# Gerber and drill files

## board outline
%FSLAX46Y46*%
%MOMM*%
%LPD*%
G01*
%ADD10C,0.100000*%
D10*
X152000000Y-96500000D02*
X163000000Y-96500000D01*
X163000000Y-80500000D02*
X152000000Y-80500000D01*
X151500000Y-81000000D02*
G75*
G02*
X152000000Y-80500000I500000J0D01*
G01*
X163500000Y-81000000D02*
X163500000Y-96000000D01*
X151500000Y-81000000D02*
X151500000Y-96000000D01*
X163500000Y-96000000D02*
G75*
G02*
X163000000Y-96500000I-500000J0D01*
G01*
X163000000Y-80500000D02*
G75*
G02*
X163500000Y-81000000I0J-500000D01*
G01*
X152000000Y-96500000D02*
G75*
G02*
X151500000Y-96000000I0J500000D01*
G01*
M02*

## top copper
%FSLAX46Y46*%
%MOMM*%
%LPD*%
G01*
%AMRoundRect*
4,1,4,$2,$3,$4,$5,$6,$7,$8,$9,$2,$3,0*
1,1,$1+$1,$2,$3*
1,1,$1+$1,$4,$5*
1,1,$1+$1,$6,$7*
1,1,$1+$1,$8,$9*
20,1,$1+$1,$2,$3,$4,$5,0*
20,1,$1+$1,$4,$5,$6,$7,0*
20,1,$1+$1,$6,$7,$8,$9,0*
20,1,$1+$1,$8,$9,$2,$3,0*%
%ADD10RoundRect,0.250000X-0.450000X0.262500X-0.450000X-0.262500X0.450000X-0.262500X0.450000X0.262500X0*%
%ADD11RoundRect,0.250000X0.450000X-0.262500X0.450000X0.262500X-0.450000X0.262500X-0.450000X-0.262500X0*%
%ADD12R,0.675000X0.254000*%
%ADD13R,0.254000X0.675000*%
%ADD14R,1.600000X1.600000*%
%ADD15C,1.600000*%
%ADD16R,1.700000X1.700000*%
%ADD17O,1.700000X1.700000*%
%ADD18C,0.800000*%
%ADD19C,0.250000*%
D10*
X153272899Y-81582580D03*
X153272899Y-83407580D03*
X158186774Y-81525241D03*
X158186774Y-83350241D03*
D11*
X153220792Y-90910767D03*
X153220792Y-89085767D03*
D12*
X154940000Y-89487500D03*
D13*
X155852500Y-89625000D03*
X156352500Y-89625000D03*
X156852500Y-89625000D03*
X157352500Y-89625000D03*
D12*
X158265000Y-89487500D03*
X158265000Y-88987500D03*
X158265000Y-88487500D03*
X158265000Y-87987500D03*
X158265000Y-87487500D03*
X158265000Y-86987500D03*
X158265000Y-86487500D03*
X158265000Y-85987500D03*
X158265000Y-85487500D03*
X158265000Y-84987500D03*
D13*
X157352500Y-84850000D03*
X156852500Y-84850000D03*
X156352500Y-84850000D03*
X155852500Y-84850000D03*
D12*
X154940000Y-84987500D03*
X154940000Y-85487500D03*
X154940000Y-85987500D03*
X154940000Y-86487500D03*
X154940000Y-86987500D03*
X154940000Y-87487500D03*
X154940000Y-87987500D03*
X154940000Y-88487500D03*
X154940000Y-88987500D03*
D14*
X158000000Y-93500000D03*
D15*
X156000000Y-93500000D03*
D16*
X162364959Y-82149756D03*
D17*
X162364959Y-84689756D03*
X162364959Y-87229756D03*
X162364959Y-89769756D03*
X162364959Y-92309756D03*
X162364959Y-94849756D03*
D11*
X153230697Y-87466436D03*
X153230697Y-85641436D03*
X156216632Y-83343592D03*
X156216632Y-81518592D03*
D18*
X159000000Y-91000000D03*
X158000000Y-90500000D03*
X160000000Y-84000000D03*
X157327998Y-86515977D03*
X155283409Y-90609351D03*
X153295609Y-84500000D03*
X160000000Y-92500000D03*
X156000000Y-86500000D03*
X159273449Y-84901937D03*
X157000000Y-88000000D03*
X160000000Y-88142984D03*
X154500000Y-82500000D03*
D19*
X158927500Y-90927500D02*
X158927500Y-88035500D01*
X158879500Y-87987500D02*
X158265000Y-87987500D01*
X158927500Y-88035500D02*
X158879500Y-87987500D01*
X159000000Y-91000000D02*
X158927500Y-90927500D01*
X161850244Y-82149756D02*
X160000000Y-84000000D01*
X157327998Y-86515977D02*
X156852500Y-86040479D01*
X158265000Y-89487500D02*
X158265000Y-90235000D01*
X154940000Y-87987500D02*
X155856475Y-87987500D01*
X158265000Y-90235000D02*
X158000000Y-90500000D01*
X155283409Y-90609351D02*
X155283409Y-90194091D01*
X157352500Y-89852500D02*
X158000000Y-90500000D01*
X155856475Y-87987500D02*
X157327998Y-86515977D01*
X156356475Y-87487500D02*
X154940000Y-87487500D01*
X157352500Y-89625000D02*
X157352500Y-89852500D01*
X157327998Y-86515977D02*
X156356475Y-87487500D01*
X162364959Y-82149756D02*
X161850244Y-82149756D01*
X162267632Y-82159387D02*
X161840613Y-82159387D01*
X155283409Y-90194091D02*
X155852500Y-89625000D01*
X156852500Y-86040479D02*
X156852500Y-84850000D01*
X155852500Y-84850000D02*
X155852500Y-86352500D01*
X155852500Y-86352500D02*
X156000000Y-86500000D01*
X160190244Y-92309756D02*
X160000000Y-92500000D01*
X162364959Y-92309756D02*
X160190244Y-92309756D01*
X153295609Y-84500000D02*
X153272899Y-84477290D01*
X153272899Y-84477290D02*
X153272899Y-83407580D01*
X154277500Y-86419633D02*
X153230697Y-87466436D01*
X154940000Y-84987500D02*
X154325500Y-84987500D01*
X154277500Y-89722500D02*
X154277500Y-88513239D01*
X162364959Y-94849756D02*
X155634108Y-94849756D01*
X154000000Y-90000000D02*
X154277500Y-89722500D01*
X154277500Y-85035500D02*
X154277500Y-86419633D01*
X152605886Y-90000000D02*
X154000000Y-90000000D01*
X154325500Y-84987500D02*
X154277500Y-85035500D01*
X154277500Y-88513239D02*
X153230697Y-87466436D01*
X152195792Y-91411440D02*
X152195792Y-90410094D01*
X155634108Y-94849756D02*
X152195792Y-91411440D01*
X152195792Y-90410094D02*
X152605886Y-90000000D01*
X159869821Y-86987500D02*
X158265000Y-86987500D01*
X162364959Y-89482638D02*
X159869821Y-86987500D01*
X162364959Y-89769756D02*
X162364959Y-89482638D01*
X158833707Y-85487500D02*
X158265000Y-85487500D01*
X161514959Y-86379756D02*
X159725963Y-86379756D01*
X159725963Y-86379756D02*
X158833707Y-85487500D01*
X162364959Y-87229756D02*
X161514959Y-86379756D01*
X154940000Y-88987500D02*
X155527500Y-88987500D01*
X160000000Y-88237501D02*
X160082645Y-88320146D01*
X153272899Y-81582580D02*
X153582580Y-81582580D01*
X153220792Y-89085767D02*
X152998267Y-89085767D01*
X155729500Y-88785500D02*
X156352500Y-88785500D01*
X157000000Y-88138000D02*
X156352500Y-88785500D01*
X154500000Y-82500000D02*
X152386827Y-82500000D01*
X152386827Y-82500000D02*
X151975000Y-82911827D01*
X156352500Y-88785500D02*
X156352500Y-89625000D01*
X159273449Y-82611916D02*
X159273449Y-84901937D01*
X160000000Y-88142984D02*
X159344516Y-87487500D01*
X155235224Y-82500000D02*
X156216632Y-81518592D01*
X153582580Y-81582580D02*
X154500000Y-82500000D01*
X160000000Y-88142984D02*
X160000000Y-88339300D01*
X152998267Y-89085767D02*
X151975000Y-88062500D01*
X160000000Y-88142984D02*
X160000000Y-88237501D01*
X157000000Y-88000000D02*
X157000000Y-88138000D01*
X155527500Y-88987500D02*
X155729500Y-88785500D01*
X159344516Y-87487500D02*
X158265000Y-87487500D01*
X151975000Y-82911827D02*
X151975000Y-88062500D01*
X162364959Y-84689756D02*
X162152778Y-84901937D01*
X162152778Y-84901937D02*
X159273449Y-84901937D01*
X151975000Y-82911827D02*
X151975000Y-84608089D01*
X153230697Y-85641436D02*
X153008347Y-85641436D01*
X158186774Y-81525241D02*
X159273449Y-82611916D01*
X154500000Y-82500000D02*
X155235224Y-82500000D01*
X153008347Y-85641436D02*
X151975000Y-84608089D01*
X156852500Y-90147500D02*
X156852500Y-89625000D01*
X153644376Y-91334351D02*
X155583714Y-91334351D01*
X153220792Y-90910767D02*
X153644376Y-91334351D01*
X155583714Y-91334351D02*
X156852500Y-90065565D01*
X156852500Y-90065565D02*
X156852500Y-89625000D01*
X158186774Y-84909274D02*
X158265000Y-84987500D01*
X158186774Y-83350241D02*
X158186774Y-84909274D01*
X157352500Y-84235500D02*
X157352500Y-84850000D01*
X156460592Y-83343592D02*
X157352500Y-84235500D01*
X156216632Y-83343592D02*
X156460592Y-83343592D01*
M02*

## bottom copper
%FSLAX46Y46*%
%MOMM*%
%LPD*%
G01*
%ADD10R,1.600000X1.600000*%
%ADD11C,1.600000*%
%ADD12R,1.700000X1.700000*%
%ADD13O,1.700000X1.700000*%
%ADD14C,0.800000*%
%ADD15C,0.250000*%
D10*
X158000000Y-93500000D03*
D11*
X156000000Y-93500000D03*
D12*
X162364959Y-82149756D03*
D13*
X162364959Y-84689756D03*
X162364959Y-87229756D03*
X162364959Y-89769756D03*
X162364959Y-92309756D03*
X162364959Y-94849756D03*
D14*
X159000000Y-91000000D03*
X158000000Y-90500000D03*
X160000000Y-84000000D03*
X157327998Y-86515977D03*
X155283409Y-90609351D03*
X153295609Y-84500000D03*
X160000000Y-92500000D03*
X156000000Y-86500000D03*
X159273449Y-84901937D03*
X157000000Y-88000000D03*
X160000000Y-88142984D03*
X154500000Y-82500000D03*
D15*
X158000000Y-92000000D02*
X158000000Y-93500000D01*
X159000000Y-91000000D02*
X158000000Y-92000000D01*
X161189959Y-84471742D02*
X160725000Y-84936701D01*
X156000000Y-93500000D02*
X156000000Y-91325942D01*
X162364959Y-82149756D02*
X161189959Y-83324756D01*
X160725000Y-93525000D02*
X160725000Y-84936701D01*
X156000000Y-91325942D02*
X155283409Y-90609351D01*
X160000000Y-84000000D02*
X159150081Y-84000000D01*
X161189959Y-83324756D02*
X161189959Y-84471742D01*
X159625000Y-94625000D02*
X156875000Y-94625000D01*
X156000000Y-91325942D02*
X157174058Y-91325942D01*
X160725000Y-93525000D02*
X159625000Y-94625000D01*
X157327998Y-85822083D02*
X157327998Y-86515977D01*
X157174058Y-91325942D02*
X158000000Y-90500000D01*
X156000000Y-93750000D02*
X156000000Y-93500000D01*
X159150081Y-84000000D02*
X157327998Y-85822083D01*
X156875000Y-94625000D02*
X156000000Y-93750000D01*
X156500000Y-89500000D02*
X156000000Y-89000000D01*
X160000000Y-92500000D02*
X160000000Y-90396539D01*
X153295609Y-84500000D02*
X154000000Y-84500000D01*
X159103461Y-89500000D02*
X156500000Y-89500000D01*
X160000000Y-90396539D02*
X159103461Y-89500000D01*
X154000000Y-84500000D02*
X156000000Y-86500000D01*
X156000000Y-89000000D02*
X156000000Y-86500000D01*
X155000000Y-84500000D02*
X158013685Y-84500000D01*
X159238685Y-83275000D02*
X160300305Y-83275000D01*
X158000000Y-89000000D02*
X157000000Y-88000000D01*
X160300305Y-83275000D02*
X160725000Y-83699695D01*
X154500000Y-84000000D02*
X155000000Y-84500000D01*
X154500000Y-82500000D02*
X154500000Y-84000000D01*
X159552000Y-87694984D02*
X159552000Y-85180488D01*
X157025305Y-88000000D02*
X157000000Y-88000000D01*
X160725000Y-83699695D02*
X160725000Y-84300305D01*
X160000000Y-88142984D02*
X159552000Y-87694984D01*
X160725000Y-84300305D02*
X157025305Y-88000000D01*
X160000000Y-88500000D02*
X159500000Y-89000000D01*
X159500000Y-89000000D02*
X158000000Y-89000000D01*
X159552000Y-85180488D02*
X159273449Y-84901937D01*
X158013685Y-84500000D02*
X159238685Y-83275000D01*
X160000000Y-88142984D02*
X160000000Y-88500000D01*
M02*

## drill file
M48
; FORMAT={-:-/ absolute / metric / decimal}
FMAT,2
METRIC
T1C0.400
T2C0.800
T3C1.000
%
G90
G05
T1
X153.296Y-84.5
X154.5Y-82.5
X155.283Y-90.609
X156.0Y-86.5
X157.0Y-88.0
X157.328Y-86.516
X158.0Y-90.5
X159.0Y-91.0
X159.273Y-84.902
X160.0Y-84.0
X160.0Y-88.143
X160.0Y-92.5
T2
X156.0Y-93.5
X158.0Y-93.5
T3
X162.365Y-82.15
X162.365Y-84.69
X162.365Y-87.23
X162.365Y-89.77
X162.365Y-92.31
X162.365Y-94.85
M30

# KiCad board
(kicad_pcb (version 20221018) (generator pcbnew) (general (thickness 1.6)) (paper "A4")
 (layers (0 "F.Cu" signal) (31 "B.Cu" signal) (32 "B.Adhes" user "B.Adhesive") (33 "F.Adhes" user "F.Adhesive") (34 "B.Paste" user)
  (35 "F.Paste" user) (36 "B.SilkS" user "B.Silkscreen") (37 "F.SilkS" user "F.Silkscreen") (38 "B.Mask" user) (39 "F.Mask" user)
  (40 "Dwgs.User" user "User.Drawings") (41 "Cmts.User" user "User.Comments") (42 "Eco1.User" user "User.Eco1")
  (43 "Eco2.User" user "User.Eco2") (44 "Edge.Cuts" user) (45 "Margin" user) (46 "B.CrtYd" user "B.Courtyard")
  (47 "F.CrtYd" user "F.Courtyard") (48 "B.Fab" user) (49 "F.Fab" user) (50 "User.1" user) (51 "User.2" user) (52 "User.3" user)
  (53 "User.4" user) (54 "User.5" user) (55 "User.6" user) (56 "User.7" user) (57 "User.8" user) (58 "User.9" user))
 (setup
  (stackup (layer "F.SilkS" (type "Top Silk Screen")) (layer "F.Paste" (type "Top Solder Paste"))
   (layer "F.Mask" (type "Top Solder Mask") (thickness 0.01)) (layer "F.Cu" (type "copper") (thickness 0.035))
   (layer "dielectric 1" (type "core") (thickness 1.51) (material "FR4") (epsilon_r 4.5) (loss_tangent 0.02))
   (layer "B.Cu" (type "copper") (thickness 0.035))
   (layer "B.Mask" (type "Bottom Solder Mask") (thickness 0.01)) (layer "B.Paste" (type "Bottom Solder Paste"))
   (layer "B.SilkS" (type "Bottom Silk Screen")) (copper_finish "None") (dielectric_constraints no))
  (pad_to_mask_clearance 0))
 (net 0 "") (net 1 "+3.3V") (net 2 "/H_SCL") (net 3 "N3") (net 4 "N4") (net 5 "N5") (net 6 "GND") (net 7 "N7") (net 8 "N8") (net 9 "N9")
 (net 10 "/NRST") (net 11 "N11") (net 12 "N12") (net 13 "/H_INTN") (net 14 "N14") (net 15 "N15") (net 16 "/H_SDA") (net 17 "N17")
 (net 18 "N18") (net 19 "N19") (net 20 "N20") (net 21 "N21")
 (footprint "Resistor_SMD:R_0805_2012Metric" (layer "F.Cu") (at 153.272899 82.49508 -90)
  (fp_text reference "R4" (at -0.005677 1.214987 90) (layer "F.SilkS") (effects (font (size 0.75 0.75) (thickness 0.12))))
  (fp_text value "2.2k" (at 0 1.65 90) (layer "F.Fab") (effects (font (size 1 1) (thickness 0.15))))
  (pad "1" smd roundrect (at -0.9125 0 270) (size 1.025 1.4) (layers "F.Cu" "F.Paste" "F.Mask") (roundrect_rratio 0.243902) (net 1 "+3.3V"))
  (pad "2" smd roundrect (at 0.9125 0 270) (size 1.025 1.4) (layers "F.Cu" "F.Paste" "F.Mask") (roundrect_rratio 0.243902) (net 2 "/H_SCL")))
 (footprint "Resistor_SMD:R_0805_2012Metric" (layer "F.Cu") (at 158.186774 82.437741 -90)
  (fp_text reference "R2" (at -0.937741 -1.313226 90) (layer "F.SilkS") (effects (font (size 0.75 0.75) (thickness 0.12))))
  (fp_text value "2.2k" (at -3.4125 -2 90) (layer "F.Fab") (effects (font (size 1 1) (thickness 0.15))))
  (pad "1" smd roundrect (at -0.9125 0 270) (size 1.025 1.4) (layers "F.Cu" "F.Paste" "F.Mask") (roundrect_rratio 0.243902) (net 1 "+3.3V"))
  (pad "2" smd roundrect (at 0.9125 0 270) (size 1.025 1.4) (layers "F.Cu" "F.Paste" "F.Mask") (roundrect_rratio 0.243902) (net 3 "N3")))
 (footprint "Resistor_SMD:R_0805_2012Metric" (layer "F.Cu") (at 153.220792 89.998267 90)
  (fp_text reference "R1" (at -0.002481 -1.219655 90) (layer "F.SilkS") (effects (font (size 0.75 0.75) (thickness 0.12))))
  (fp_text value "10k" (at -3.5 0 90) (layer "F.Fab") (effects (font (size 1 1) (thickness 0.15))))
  (pad "1" smd roundrect (at -0.9125 0 90) (size 1.025 1.4) (layers "F.Cu" "F.Paste" "F.Mask") (roundrect_rratio 0.243902) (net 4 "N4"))
  (pad "2" smd roundrect (at 0.9125 0 90) (size 1.025 1.4) (layers "F.Cu" "F.Paste" "F.Mask") (roundrect_rratio 0.243902) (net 1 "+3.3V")))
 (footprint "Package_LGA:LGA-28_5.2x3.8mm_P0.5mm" (layer "F.Cu") (at 156.6025 87.2375 90)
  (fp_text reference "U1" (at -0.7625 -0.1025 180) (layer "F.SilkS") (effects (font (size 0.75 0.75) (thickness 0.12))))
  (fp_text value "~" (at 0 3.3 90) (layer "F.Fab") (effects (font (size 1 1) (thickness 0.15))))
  (pad "1" smd rect (at -2.25 -1.6625 90) (size 0.254 0.675) (layers "F.Cu" "F.Paste" "F.Mask") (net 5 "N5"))
  (pad "2" smd rect (at -2.3875 -0.75 180) (size 0.254 0.675) (layers "F.Cu" "F.Paste" "F.Mask") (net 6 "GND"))
  (pad "3" smd rect (at -2.3875 -0.25 180) (size 0.254 0.675) (layers "F.Cu" "F.Paste" "F.Mask") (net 1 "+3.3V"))
  (pad "4" smd rect (at -2.3875 0.25 180) (size 0.254 0.675) (layers "F.Cu" "F.Paste" "F.Mask") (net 4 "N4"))
  (pad "5" smd rect (at -2.3875 0.75 180) (size 0.254 0.675) (layers "F.Cu" "F.Paste" "F.Mask") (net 6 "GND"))
  (pad "6" smd rect (at -2.25 1.6625 90) (size 0.254 0.675) (layers "F.Cu" "F.Paste" "F.Mask") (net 6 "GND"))
  (pad "7" smd rect (at -1.75 1.6625 90) (size 0.254 0.675) (layers "F.Cu" "F.Paste" "F.Mask") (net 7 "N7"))
  (pad "8" smd rect (at -1.25 1.6625 90) (size 0.254 0.675) (layers "F.Cu" "F.Paste" "F.Mask") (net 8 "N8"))
  (pad "9" smd rect (at -0.75 1.6625 90) (size 0.254 0.675) (layers "F.Cu" "F.Paste" "F.Mask") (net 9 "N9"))
  (pad "10" smd rect (at -0.25 1.6625 90) (size 0.254 0.675) (layers "F.Cu" "F.Paste" "F.Mask") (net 1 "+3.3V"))
  (pad "11" smd rect (at 0.25 1.6625 90) (size 0.254 0.675) (layers "F.Cu" "F.Paste" "F.Mask") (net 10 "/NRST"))
  (pad "12" smd rect (at 0.75 1.6625 90) (size 0.254 0.675) (layers "F.Cu" "F.Paste" "F.Mask") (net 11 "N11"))
  (pad "13" smd rect (at 1.25 1.6625 90) (size 0.254 0.675) (layers "F.Cu" "F.Paste" "F.Mask") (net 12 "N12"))
  (pad "14" smd rect (at 1.75 1.6625 90) (size 0.254 0.675) (layers "F.Cu" "F.Paste" "F.Mask") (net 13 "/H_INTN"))
  (pad "15" smd rect (at 2.25 1.6625 90) (size 0.254 0.675) (layers "F.Cu" "F.Paste" "F.Mask") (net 3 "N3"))
  (pad "16" smd rect (at 2.3875 0.75 180) (size 0.254 0.675) (layers "F.Cu" "F.Paste" "F.Mask") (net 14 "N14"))
  (pad "17" smd rect (at 2.3875 0.25 180) (size 0.254 0.675) (layers "F.Cu" "F.Paste" "F.Mask") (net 6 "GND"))
  (pad "18" smd rect (at 2.3875 -0.25 180) (size 0.254 0.675) (layers "F.Cu" "F.Paste" "F.Mask") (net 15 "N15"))
  (pad "19" smd rect (at 2.3875 -0.75 180) (size 0.254 0.675) (layers "F.Cu" "F.Paste" "F.Mask") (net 2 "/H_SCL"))
  (pad "20" smd rect (at 2.25 -1.6625 90) (size 0.254 0.675) (layers "F.Cu" "F.Paste" "F.Mask") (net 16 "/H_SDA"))
  (pad "21" smd rect (at 1.75 -1.6625 90) (size 0.254 0.675) (layers "F.Cu" "F.Paste" "F.Mask") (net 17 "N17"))
  (pad "22" smd rect (at 1.25 -1.6625 90) (size 0.254 0.675) (layers "F.Cu" "F.Paste" "F.Mask") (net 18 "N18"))
  (pad "23" smd rect (at 0.75 -1.6625 90) (size 0.254 0.675) (layers "F.Cu" "F.Paste" "F.Mask") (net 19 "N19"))
  (pad "24" smd rect (at 0.25 -1.6625 90) (size 0.254 0.675) (layers "F.Cu" "F.Paste" "F.Mask") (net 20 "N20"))
  (pad "25" smd rect (at -0.25 -1.6625 90) (size 0.254 0.675) (layers "F.Cu" "F.Paste" "F.Mask") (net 6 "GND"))
  (pad "26" smd rect (at -0.75 -1.6625 90) (size 0.254 0.675) (layers "F.Cu" "F.Paste" "F.Mask") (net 6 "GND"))
  (pad "27" smd rect (at -1.25 -1.6625 90) (size 0.254 0.675) (layers "F.Cu" "F.Paste" "F.Mask") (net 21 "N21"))
  (pad "28" smd rect (at -1.75 -1.6625 90) (size 0.254 0.675) (layers "F.Cu" "F.Paste" "F.Mask") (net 1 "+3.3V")))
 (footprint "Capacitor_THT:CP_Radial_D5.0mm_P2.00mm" (layer "F.Cu") (at 158 93.5 180)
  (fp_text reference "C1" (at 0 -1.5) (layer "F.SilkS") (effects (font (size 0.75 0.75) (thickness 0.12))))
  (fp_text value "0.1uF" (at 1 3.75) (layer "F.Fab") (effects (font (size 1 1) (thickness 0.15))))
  (pad "1" thru_hole rect (at 0 0 180) (size 1.6 1.6) (drill 0.8) (layers "*.Cu" "*.Mask") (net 9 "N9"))
  (pad "2" thru_hole circle (at 2 0 180) (size 1.6 1.6) (drill 0.8) (layers "*.Cu" "*.Mask") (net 6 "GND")))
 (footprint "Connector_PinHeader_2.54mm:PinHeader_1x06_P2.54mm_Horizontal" (layer "F.Cu") (at 162.364959 82.149756)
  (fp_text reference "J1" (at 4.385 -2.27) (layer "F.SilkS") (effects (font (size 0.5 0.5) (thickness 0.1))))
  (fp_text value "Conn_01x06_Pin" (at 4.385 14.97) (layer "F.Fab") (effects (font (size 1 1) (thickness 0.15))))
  (pad "1" thru_hole rect (at 0 0) (size 1.7 1.7) (drill 1) (layers "*.Cu" "*.Mask") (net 6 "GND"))
  (pad "2" thru_hole oval (at 0 2.54) (size 1.7 1.7) (drill 1) (layers "*.Cu" "*.Mask") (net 1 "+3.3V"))
  (pad "3" thru_hole oval (at 0 5.08) (size 1.7 1.7) (drill 1) (layers "*.Cu" "*.Mask") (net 13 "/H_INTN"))
  (pad "4" thru_hole oval (at 0 7.62) (size 1.7 1.7) (drill 1) (layers "*.Cu" "*.Mask") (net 10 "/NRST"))
  (pad "5" thru_hole oval (at 0 10.16) (size 1.7 1.7) (drill 1) (layers "*.Cu" "*.Mask") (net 2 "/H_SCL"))
  (pad "6" thru_hole oval (at 0 12.7) (size 1.7 1.7) (drill 1) (layers "*.Cu" "*.Mask") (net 16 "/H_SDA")))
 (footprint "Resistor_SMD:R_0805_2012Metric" (layer "F.Cu") (at 153.230697 86.553936 90)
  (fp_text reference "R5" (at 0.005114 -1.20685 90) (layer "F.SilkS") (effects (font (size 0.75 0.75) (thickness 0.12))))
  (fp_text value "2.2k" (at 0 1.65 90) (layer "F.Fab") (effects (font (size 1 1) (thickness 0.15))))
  (pad "1" smd roundrect (at -0.9125 0 90) (size 1.025 1.4) (layers "F.Cu" "F.Paste" "F.Mask") (roundrect_rratio 0.243902) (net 16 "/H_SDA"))
  (pad "2" smd roundrect (at 0.9125 0 90) (size 1.025 1.4) (layers "F.Cu" "F.Paste" "F.Mask") (roundrect_rratio 0.243902) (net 1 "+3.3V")))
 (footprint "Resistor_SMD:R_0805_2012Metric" (layer "F.Cu") (at 156.216632 82.431092 90)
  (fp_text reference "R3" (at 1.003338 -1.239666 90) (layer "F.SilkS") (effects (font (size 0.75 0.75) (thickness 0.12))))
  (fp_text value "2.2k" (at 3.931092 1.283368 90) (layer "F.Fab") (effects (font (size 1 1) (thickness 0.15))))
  (pad "1" smd roundrect (at -0.9125 0 90) (size 1.025 1.4) (layers "F.Cu" "F.Paste" "F.Mask") (roundrect_rratio 0.243902) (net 14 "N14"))
  (pad "2" smd roundrect (at 0.9125 0 90) (size 1.025 1.4) (layers "F.Cu" "F.Paste" "F.Mask") (roundrect_rratio 0.243902) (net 1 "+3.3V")))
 (gr_line (start 152 96.5) (end 163 96.5) (stroke (width 0.1) (type default)) (layer "Edge.Cuts"))
 (gr_line (start 163 80.5) (end 152 80.5) (stroke (width 0.1) (type default)) (layer "Edge.Cuts"))
 (gr_arc (start 151.5 81) (mid 151.646447 80.646447) (end 152 80.5) (stroke (width 0.1) (type default)) (layer "Edge.Cuts"))
 (gr_line (start 163.5 81) (end 163.5 96) (stroke (width 0.1) (type default)) (layer "Edge.Cuts"))
 (gr_line (start 151.5 81) (end 151.5 96) (stroke (width 0.1) (type default)) (layer "Edge.Cuts"))
 (gr_arc (start 163.5 96) (mid 163.353553 96.353553) (end 163 96.5) (stroke (width 0.1) (type default)) (layer "Edge.Cuts"))
 (gr_arc (start 163 80.5) (mid 163.353553 80.646447) (end 163.5 81) (stroke (width 0.1) (type default)) (layer "Edge.Cuts"))
 (gr_arc (start 152 96.5) (mid 151.646447 96.353553) (end 151.5 96) (stroke (width 0.1) (type default)) (layer "Edge.Cuts"))
 (segment (start 158.9275 90.9275) (end 158.9275 88.0355) (width 0.25) (layer "F.Cu") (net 9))
 (segment (start 158.8795 87.9875) (end 158.265 87.9875) (width 0.25) (layer "F.Cu") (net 9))
 (segment (start 158.9275 88.0355) (end 158.8795 87.9875) (width 0.25) (layer "F.Cu") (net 9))
 (segment (start 159 91) (end 158.9275 90.9275) (width 0.25) (layer "F.Cu") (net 9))
 (via (at 159 91) (size 0.8) (drill 0.4) (layers "F.Cu" "B.Cu") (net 9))
 (segment (start 158 92) (end 158 93.5) (width 0.25) (layer "B.Cu") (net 9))
 (segment (start 159 91) (end 158 92) (width 0.25) (layer "B.Cu") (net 9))
 (segment (start 161.850244 82.149756) (end 160 84) (width 0.25) (layer "F.Cu") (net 6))
 (segment (start 157.327998 86.515977) (end 156.8525 86.040479) (width 0.25) (layer "F.Cu") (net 6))
 (segment (start 158.265 89.4875) (end 158.265 90.235) (width 0.25) (layer "F.Cu") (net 6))
 (segment (start 154.94 87.9875) (end 155.856475 87.9875) (width 0.25) (layer "F.Cu") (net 6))
 (segment (start 158.265 90.235) (end 158 90.5) (width 0.25) (layer "F.Cu") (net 6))
 (segment (start 155.283409 90.609351) (end 155.283409 90.194091) (width 0.25) (layer "F.Cu") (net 6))
 (segment (start 157.3525 89.8525) (end 158 90.5) (width 0.25) (layer "F.Cu") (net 6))
 (segment (start 155.856475 87.9875) (end 157.327998 86.515977) (width 0.25) (layer "F.Cu") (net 6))
 (segment (start 156.356475 87.4875) (end 154.94 87.4875) (width 0.25) (layer "F.Cu") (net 6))
 (segment (start 157.3525 89.625) (end 157.3525 89.8525) (width 0.25) (layer "F.Cu") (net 6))
 (segment (start 157.327998 86.515977) (end 156.356475 87.4875) (width 0.25) (layer "F.Cu") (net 6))
 (segment (start 162.364959 82.149756) (end 161.850244 82.149756) (width 0.25) (layer "F.Cu") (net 6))
 (segment (start 162.267632 82.159387) (end 161.840613 82.159387) (width 0.25) (layer "F.Cu") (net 6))
 (segment (start 155.283409 90.194091) (end 155.8525 89.625) (width 0.25) (layer "F.Cu") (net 6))
 (segment (start 156.8525 86.040479) (end 156.8525 84.85) (width 0.25) (layer "F.Cu") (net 6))
 (via (at 158 90.5) (size 0.8) (drill 0.4) (layers "F.Cu" "B.Cu") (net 6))
 (via (at 160 84) (size 0.8) (drill 0.4) (layers "F.Cu" "B.Cu") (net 6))
 (via (at 157.327998 86.515977) (size 0.8) (drill 0.4) (layers "F.Cu" "B.Cu") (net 6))
 (via (at 155.283409 90.609351) (size 0.8) (drill 0.4) (layers "F.Cu" "B.Cu") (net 6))
 (segment (start 161.189959 84.471742) (end 160.725 84.936701) (width 0.25) (layer "B.Cu") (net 6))
 (segment (start 156 93.5) (end 156 91.325942) (width 0.25) (layer "B.Cu") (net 6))
 (segment (start 162.364959 82.149756) (end 161.189959 83.324756) (width 0.25) (layer "B.Cu") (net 6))
 (segment (start 160.725 93.525) (end 160.725 84.936701) (width 0.25) (layer "B.Cu") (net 6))
 (segment (start 156 91.325942) (end 155.283409 90.609351) (width 0.25) (layer "B.Cu") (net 6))
 (segment (start 160 84) (end 159.150081 84) (width 0.25) (layer "B.Cu") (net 6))
 (segment (start 161.189959 83.324756) (end 161.189959 84.471742) (width 0.25) (layer "B.Cu") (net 6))
 (segment (start 159.625 94.625) (end 156.875 94.625) (width 0.25) (layer "B.Cu") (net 6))
 (segment (start 156 91.325942) (end 157.174058 91.325942) (width 0.25) (layer "B.Cu") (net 6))
 (segment (start 160.725 93.525) (end 159.625 94.625) (width 0.25) (layer "B.Cu") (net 6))
 (segment (start 157.327998 85.822083) (end 157.327998 86.515977) (width 0.25) (layer "B.Cu") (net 6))
 (segment (start 157.174058 91.325942) (end 158 90.5) (width 0.25) (layer "B.Cu") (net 6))
 (segment (start 156 93.75) (end 156 93.5) (width 0.25) (layer "B.Cu") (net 6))
 (segment (start 159.150081 84) (end 157.327998 85.822083) (width 0.25) (layer "B.Cu") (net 6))
 (segment (start 156.875 94.625) (end 156 93.75) (width 0.25) (layer "B.Cu") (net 6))
 (segment (start 155.8525 84.85) (end 155.8525 86.3525) (width 0.25) (layer "F.Cu") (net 2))
 (segment (start 155.8525 86.3525) (end 156 86.5) (width 0.25) (layer "F.Cu") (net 2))
 (segment (start 160.190244 92.309756) (end 160 92.5) (width 0.25) (layer "F.Cu") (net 2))
 (segment (start 162.364959 92.309756) (end 160.190244 92.309756) (width 0.25) (layer "F.Cu") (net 2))
 (segment (start 153.295609 84.5) (end 153.272899 84.47729) (width 0.25) (layer "F.Cu") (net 2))
 (segment (start 153.272899 84.47729) (end 153.272899 83.40758) (width 0.25) (layer "F.Cu") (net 2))
 (via (at 153.295609 84.5) (size 0.8) (drill 0.4) (layers "F.Cu" "B.Cu") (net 2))
 (via (at 160 92.5) (size 0.8) (drill 0.4) (layers "F.Cu" "B.Cu") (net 2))
 (via (at 156 86.5) (size 0.8) (drill 0.4) (layers "F.Cu" "B.Cu") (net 2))
 (segment (start 156.5 89.5) (end 156 89) (width 0.25) (layer "B.Cu") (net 2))
 (segment (start 160 92.5) (end 160 90.396539) (width 0.25) (layer "B.Cu") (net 2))
 (segment (start 153.295609 84.5) (end 154 84.5) (width 0.25) (layer "B.Cu") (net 2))
 (segment (start 159.103461 89.5) (end 156.5 89.5) (width 0.25) (layer "B.Cu") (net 2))
 (segment (start 160 90.396539) (end 159.103461 89.5) (width 0.25) (layer "B.Cu") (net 2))
 (segment (start 154 84.5) (end 156 86.5) (width 0.25) (layer "B.Cu") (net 2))
 (segment (start 156 89) (end 156 86.5) (width 0.25) (layer "B.Cu") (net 2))
 (segment (start 154.2775 86.419633) (end 153.230697 87.466436) (width 0.25) (layer "F.Cu") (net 16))
 (segment (start 154.94 84.9875) (end 154.3255 84.9875) (width 0.25) (layer "F.Cu") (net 16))
 (segment (start 154.2775 89.7225) (end 154.2775 88.513239) (width 0.25) (layer "F.Cu") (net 16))
 (segment (start 162.364959 94.849756) (end 155.634108 94.849756) (width 0.25) (layer "F.Cu") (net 16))
 (segment (start 154 90) (end 154.2775 89.7225) (width 0.25) (layer "F.Cu") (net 16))
 (segment (start 154.2775 85.0355) (end 154.2775 86.419633) (width 0.25) (layer "F.Cu") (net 16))
 (segment (start 152.605886 90) (end 154 90) (width 0.25) (layer "F.Cu") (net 16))
 (segment (start 154.3255 84.9875) (end 154.2775 85.0355) (width 0.25) (layer "F.Cu") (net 16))
 (segment (start 154.2775 88.513239) (end 153.230697 87.466436) (width 0.25) (layer "F.Cu") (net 16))
 (segment (start 152.195792 91.41144) (end 152.195792 90.410094) (width 0.25) (layer "F.Cu") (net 16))
 (segment (start 155.634108 94.849756) (end 152.195792 91.41144) (width 0.25) (layer "F.Cu") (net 16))
 (segment (start 152.195792 90.410094) (end 152.605886 90) (width 0.25) (layer "F.Cu") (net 16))
 (segment (start 159.869821 86.9875) (end 158.265 86.9875) (width 0.25) (layer "F.Cu") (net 10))
 (segment (start 162.364959 89.482638) (end 159.869821 86.9875) (width 0.25) (layer "F.Cu") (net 10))
 (segment (start 162.364959 89.769756) (end 162.364959 89.482638) (width 0.25) (layer "F.Cu") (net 10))
 (segment (start 158.833707 85.4875) (end 158.265 85.4875) (width 0.25) (layer "F.Cu") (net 13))
 (segment (start 161.514959 86.379756) (end 159.725963 86.379756) (width 0.25) (layer "F.Cu") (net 13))
 (segment (start 159.725963 86.379756) (end 158.833707 85.4875) (width 0.25) (layer "F.Cu") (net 13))
 (segment (start 162.364959 87.229756) (end 161.514959 86.379756) (width 0.25) (layer "F.Cu") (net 13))
 (segment (start 154.94 88.9875) (end 155.5275 88.9875) (width 0.25) (layer "F.Cu") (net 1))
 (segment (start 160 88.237501) (end 160.082645 88.320146) (width 0.25) (layer "F.Cu") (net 1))
 (segment (start 153.272899 81.58258) (end 153.58258 81.58258) (width 0.25) (layer "F.Cu") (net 1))
 (segment (start 153.220792 89.085767) (end 152.998267 89.085767) (width 0.25) (layer "F.Cu") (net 1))
 (segment (start 155.7295 88.7855) (end 156.3525 88.7855) (width 0.25) (layer "F.Cu") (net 1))
 (segment (start 157 88.138) (end 156.3525 88.7855) (width 0.25) (layer "F.Cu") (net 1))
 (segment (start 154.5 82.5) (end 152.386827 82.5) (width 0.25) (layer "F.Cu") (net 1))
 (segment (start 152.386827 82.5) (end 151.975 82.911827) (width 0.25) (layer "F.Cu") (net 1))
 (segment (start 156.3525 88.7855) (end 156.3525 89.625) (width 0.25) (layer "F.Cu") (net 1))
 (segment (start 159.273449 82.611916) (end 159.273449 84.901937) (width 0.25) (layer "F.Cu") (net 1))
 (segment (start 160 88.142984) (end 159.344516 87.4875) (width 0.25) (layer "F.Cu") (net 1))
 (segment (start 155.235224 82.5) (end 156.216632 81.518592) (width 0.25) (layer "F.Cu") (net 1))
 (segment (start 153.58258 81.58258) (end 154.5 82.5) (width 0.25) (layer "F.Cu") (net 1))
 (segment (start 160 88.142984) (end 160 88.3393) (width 0.25) (layer "F.Cu") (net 1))
 (segment (start 152.998267 89.085767) (end 151.975 88.0625) (width 0.25) (layer "F.Cu") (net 1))
 (segment (start 160 88.142984) (end 160 88.237501) (width 0.25) (layer "F.Cu") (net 1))
 (segment (start 157 88) (end 157 88.138) (width 0.25) (layer "F.Cu") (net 1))
 (segment (start 155.5275 88.9875) (end 155.7295 88.7855) (width 0.25) (layer "F.Cu") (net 1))
 (segment (start 159.344516 87.4875) (end 158.265 87.4875) (width 0.25) (layer "F.Cu") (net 1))
 (segment (start 151.975 82.911827) (end 151.975 88.0625) (width 0.25) (layer "F.Cu") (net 1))
 (segment (start 162.364959 84.689756) (end 162.152778 84.901937) (width 0.25) (layer "F.Cu") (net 1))
 (segment (start 162.152778 84.901937) (end 159.273449 84.901937) (width 0.25) (layer "F.Cu") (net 1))
 (segment (start 151.975 82.911827) (end 151.975 84.608089) (width 0.25) (layer "F.Cu") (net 1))
 (segment (start 153.230697 85.641436) (end 153.008347 85.641436) (width 0.25) (layer "F.Cu") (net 1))
 (segment (start 158.186774 81.525241) (end 159.273449 82.611916) (width 0.25) (layer "F.Cu") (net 1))
 (segment (start 154.5 82.5) (end 155.235224 82.5) (width 0.25) (layer "F.Cu") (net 1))
 (segment (start 153.008347 85.641436) (end 151.975 84.608089) (width 0.25) (layer "F.Cu") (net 1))
 (via (at 159.273449 84.901937) (size 0.8) (drill 0.4) (layers "F.Cu" "B.Cu") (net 1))
 (via (at 157 88) (size 0.8) (drill 0.4) (layers "F.Cu" "B.Cu") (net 1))
 (via (at 160 88.142984) (size 0.8) (drill 0.4) (layers "F.Cu" "B.Cu") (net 1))
 (via (at 154.5 82.5) (size 0.8) (drill 0.4) (layers "F.Cu" "B.Cu") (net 1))
 (segment (start 155 84.5) (end 158.013685 84.5) (width 0.25) (layer "B.Cu") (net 1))
 (segment (start 159.238685 83.275) (end 160.300305 83.275) (width 0.25) (layer "B.Cu") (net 1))
 (segment (start 158 89) (end 157 88) (width 0.25) (layer "B.Cu") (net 1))
 (segment (start 160.300305 83.275) (end 160.725 83.699695) (width 0.25) (layer "B.Cu") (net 1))
 (segment (start 154.5 84) (end 155 84.5) (width 0.25) (layer "B.Cu") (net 1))
 (segment (start 154.5 82.5) (end 154.5 84) (width 0.25) (layer "B.Cu") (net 1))
 (segment (start 159.552 87.694984) (end 159.552 85.180488) (width 0.25) (layer "B.Cu") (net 1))
 (segment (start 157.025305 88) (end 157 88) (width 0.25) (layer "B.Cu") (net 1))
 (segment (start 160.725 83.699695) (end 160.725 84.300305) (width 0.25) (layer "B.Cu") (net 1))
 (segment (start 160 88.142984) (end 159.552 87.694984) (width 0.25) (layer "B.Cu") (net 1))
 (segment (start 160.725 84.300305) (end 157.025305 88) (width 0.25) (layer "B.Cu") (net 1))
 (segment (start 160 88.5) (end 159.5 89) (width 0.25) (layer "B.Cu") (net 1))
 (segment (start 159.5 89) (end 158 89) (width 0.25) (layer "B.Cu") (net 1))
 (segment (start 159.552 85.180488) (end 159.273449 84.901937) (width 0.25) (layer "B.Cu") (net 1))
 (segment (start 158.013685 84.5) (end 159.238685 83.275) (width 0.25) (layer "B.Cu") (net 1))
 (segment (start 160 88.142984) (end 160 88.5) (width 0.25) (layer "B.Cu") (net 1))
 (segment (start 156.8525 90.1475) (end 156.8525 89.625) (width 0.25) (layer "F.Cu") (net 4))
 (segment (start 153.644376 91.334351) (end 155.583714 91.334351) (width 0.25) (layer "F.Cu") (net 4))
 (segment (start 153.220792 90.910767) (end 153.644376 91.334351) (width 0.25) (layer "F.Cu") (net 4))
 (segment (start 155.583714 91.334351) (end 156.8525 90.065565) (width 0.25) (layer "F.Cu") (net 4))
 (segment (start 156.8525 90.065565) (end 156.8525 89.625) (width 0.25) (layer "F.Cu") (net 4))
 (segment (start 158.186774 84.909274) (end 158.265 84.9875) (width 0.25) (layer "F.Cu") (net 3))
 (segment (start 158.186774 83.350241) (end 158.186774 84.909274) (width 0.25) (layer "F.Cu") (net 3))
 (segment (start 157.3525 84.2355) (end 157.3525 84.85) (width 0.25) (layer "F.Cu") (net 14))
 (segment (start 156.460592 83.343592) (end 157.3525 84.2355) (width 0.25) (layer "F.Cu") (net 14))
 (segment (start 156.216632 83.343592) (end 156.460592 83.343592) (width 0.25) (layer "F.Cu") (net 14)))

